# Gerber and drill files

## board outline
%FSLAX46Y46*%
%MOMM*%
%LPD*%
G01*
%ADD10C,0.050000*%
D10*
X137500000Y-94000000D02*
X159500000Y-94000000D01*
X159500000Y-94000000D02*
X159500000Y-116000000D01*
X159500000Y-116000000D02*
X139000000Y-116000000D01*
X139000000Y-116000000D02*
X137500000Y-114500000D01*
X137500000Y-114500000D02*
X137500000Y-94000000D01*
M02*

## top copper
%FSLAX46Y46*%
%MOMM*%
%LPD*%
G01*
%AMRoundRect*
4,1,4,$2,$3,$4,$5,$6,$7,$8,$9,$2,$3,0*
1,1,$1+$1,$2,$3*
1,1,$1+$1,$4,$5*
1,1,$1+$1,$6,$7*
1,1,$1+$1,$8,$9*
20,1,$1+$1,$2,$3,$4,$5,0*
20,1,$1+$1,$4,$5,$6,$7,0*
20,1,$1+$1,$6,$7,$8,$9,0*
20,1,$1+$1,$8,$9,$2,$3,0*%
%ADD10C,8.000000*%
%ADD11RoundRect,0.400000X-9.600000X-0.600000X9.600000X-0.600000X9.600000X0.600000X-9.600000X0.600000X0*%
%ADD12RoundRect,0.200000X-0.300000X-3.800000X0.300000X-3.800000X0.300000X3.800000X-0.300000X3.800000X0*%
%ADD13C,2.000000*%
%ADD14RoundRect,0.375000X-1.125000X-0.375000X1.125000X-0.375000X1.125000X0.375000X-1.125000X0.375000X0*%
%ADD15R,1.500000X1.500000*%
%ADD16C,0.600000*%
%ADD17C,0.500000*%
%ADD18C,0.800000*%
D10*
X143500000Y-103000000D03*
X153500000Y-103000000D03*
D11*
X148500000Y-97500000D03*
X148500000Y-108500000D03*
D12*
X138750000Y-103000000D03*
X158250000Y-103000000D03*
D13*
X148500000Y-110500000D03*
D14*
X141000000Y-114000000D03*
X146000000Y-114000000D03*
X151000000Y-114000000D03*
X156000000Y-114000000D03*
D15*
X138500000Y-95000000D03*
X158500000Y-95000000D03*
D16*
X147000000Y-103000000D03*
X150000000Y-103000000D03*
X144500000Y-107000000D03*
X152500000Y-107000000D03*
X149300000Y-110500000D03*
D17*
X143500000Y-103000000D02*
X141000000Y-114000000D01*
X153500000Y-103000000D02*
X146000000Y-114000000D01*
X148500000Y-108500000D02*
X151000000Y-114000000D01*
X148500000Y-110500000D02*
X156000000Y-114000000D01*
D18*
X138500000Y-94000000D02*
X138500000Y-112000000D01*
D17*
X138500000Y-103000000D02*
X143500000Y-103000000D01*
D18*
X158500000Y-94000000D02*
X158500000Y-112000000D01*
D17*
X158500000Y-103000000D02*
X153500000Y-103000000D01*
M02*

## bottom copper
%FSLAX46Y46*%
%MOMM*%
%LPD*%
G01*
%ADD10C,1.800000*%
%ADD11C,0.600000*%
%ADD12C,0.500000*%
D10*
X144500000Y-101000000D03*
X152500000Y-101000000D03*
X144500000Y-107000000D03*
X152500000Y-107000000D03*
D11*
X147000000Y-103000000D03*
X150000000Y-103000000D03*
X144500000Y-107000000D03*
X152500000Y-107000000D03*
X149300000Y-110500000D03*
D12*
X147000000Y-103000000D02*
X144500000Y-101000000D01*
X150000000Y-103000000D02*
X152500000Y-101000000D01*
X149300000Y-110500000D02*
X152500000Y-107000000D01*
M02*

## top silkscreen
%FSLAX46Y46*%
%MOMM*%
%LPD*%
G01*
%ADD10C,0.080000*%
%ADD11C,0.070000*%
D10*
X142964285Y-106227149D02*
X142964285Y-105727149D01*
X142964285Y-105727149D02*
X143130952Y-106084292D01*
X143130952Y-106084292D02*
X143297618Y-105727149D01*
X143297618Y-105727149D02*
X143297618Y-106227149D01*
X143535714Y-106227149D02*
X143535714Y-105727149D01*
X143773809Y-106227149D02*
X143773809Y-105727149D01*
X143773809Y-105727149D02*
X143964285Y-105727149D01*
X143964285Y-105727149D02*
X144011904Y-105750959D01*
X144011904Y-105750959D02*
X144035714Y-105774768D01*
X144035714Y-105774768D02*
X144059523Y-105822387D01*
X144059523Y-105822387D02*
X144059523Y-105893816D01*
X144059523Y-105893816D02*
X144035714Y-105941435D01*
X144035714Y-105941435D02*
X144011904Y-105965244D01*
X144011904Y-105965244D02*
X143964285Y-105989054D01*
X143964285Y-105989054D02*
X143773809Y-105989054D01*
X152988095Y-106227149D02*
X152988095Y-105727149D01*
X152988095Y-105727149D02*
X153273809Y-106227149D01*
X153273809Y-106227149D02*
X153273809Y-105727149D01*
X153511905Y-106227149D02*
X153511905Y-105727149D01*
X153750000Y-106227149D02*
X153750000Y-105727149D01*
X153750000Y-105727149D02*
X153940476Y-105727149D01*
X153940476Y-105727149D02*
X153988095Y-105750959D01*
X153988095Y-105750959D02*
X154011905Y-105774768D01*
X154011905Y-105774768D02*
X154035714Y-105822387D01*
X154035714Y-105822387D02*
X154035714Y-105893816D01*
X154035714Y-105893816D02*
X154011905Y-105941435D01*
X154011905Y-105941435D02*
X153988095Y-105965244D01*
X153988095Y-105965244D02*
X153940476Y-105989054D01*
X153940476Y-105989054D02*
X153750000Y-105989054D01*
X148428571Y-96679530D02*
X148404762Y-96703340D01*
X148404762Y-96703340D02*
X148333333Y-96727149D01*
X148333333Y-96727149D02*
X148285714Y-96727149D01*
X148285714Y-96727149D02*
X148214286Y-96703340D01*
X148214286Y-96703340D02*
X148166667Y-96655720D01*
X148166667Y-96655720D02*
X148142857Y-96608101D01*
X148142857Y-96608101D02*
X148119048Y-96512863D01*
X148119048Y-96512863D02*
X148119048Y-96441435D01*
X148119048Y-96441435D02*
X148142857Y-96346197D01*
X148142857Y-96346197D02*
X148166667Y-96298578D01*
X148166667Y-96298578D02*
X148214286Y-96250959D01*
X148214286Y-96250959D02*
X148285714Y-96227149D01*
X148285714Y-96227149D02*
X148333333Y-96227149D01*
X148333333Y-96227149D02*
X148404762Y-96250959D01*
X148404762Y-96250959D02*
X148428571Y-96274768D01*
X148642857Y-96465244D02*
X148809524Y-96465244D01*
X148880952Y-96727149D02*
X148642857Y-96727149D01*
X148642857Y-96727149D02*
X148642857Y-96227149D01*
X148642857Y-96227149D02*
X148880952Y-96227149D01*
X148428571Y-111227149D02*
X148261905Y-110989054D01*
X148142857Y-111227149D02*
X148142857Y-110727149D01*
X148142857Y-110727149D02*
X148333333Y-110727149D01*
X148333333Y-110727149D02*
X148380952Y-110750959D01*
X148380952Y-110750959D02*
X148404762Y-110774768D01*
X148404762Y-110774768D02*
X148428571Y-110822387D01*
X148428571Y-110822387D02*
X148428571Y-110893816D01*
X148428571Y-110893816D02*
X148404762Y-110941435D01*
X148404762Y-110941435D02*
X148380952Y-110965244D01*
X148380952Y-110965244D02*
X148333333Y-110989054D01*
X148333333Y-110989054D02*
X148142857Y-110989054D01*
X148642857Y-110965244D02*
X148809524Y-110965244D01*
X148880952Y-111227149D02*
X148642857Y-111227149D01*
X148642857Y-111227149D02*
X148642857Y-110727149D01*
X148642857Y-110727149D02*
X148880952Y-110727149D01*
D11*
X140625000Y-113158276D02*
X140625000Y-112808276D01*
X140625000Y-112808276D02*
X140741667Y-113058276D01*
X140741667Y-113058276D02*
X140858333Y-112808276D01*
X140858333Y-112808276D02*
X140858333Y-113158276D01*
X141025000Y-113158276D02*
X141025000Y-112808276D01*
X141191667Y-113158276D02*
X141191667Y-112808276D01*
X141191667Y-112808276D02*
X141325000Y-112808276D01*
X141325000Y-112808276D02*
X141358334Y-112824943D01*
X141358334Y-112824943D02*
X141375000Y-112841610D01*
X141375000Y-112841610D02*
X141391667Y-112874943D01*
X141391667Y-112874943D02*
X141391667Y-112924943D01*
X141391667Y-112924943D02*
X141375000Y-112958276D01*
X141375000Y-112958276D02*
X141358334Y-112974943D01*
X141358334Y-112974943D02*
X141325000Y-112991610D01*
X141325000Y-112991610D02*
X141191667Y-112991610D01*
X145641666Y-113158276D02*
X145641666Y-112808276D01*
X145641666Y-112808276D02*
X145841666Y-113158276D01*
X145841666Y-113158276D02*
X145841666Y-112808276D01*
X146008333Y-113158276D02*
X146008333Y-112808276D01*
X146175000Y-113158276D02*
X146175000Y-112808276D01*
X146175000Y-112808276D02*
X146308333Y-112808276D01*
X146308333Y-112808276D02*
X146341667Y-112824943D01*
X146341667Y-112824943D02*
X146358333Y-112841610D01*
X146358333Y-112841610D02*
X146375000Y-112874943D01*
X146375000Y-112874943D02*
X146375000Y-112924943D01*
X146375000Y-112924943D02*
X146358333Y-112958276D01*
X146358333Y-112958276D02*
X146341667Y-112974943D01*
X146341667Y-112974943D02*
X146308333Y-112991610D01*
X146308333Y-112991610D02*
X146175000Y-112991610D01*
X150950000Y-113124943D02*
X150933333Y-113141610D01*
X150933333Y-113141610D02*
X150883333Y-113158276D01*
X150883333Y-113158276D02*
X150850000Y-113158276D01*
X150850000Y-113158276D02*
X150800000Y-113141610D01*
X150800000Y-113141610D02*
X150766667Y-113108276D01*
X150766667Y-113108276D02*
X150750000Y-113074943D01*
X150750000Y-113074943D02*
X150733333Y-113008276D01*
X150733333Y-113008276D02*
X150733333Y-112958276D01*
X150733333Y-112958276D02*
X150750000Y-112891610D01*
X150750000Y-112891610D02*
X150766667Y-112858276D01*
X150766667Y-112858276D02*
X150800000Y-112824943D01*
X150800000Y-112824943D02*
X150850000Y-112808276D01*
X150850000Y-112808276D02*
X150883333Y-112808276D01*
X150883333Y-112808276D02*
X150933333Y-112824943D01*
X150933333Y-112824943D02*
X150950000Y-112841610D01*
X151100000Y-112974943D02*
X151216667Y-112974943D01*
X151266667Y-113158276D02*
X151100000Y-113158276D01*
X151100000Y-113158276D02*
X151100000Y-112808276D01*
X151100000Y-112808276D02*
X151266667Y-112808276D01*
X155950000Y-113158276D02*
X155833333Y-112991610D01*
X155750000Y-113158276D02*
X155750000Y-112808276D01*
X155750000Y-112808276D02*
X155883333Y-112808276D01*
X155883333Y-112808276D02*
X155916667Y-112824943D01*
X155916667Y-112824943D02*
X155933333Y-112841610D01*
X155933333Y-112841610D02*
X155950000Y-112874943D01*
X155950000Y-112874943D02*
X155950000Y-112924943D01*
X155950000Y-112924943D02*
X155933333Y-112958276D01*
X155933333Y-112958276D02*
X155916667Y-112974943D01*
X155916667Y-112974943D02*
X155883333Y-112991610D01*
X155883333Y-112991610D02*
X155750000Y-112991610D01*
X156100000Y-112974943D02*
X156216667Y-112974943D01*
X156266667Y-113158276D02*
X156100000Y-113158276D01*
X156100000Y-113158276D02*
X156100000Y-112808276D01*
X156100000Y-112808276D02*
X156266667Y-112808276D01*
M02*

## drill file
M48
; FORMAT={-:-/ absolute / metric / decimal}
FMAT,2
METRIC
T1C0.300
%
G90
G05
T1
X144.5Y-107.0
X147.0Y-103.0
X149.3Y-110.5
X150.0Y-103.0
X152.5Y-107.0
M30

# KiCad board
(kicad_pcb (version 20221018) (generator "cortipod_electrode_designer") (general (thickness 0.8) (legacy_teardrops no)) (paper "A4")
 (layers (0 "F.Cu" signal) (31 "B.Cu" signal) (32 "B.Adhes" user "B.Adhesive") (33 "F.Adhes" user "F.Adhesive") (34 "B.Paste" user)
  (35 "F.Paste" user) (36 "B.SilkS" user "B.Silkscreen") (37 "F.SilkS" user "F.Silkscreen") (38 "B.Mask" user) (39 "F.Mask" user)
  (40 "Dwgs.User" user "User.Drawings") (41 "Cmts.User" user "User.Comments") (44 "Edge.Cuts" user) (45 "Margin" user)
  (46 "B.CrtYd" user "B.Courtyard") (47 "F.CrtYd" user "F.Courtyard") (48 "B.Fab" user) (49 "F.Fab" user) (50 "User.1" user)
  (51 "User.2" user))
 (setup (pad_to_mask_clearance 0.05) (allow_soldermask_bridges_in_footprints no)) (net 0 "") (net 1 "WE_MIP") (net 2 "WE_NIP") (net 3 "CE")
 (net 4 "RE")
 (gr_line (start 137.5 94) (end 159.5 94) (layer "Edge.Cuts") (width 0.05))
 (gr_line (start 159.5 94) (end 159.5 116) (layer "Edge.Cuts") (width 0.05))
 (gr_line (start 159.5 116) (end 139 116) (layer "Edge.Cuts") (width 0.05))
 (gr_line (start 139 116) (end 137.5 114.5) (layer "Edge.Cuts") (width 0.05))
 (gr_line (start 137.5 114.5) (end 137.5 94) (layer "Edge.Cuts") (width 0.05))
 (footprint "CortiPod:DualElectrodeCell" (layer "F.Cu") (at 148.5 103)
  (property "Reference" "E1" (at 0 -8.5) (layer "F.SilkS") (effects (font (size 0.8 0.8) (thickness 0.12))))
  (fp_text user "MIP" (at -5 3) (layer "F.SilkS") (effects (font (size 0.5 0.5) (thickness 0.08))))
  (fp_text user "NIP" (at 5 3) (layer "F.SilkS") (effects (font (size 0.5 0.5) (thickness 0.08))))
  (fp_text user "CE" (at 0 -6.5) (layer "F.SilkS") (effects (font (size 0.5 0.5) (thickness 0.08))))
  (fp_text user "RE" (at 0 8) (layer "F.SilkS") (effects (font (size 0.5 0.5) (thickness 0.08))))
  (pad "1" smd circle (at -5 0) (size 8 8) (layers "F.Cu" "F.Mask") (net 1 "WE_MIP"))
  (pad "2" smd circle (at 5 0) (size 8 8) (layers "F.Cu" "F.Mask") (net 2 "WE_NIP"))
  (pad "3T" smd roundrect (at 0 -5.5) (size 20 2) (layers "F.Cu" "F.Mask") (roundrect_rratio 0.2) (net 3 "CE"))
  (pad "3B" smd roundrect (at 0 5.5) (size 20 2) (layers "F.Cu" "F.Mask") (roundrect_rratio 0.2) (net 3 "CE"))
  (pad "3L" smd roundrect (at -9.75 0) (size 1 8) (layers "F.Cu" "F.Mask") (roundrect_rratio 0.2) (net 3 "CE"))
  (pad "3R" smd roundrect (at 9.75 0) (size 1 8) (layers "F.Cu" "F.Mask") (roundrect_rratio 0.2) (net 3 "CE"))
  (pad "4" smd circle (at 0 7.5) (size 2 2) (layers "F.Cu" "F.Mask" "F.Paste") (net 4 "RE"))
  (pad "5" smd circle (at -4 -2) (size 1.8 1.8) (layers "B.Cu" "B.Mask") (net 1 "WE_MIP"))
  (pad "6" smd circle (at 4 -2) (size 1.8 1.8) (layers "B.Cu" "B.Mask") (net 2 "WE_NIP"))
  (pad "7" smd circle (at -4 4) (size 1.8 1.8) (layers "B.Cu" "B.Mask") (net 3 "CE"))
  (pad "8" smd circle (at 4 4) (size 1.8 1.8) (layers "B.Cu" "B.Mask") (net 4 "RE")))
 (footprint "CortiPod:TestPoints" (layer "F.Cu") (at 148.5 114)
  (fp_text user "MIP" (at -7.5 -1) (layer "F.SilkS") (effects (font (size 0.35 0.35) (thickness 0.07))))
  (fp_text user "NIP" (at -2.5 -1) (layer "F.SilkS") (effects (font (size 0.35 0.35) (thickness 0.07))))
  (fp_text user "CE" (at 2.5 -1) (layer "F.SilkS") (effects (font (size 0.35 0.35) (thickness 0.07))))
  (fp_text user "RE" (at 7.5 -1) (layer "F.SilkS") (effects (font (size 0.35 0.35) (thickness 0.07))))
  (pad "TP1" smd roundrect (at -7.5 0) (size 3 1.5) (layers "F.Cu" "F.Mask") (roundrect_rratio 0.25) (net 1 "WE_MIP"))
  (pad "TP2" smd roundrect (at -2.5 0) (size 3 1.5) (layers "F.Cu" "F.Mask") (roundrect_rratio 0.25) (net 2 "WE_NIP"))
  (pad "TP3" smd roundrect (at 2.5 0) (size 3 1.5) (layers "F.Cu" "F.Mask") (roundrect_rratio 0.25) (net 3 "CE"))
  (pad "TP4" smd roundrect (at 7.5 0) (size 3 1.5) (layers "F.Cu" "F.Mask") (roundrect_rratio 0.25) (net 4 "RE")))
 (via (at 147 103) (size 0.6) (drill 0.3) (layers "F.Cu" "B.Cu") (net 1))
 (via (at 150 103) (size 0.6) (drill 0.3) (layers "F.Cu" "B.Cu") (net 2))
 (via (at 144.5 107) (size 0.6) (drill 0.3) (layers "F.Cu" "B.Cu") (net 3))
 (via (at 152.5 107) (size 0.6) (drill 0.3) (layers "F.Cu" "B.Cu") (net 3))
 (via (at 149.3 110.5) (size 0.6) (drill 0.3) (layers "F.Cu" "B.Cu") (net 4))
 (segment (start 147 103) (end 144.5 101) (width 0.5) (layer "B.Cu") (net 1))
 (segment (start 150 103) (end 152.5 101) (width 0.5) (layer "B.Cu") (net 2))
 (segment (start 149.3 110.5) (end 152.5 107) (width 0.5) (layer "B.Cu") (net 4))
 (segment (start 143.5 103) (end 141 114) (width 0.5) (layer "F.Cu") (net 1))
 (segment (start 153.5 103) (end 146 114) (width 0.5) (layer "F.Cu") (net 2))
 (segment (start 148.5 108.5) (end 151 114) (width 0.5) (layer "F.Cu") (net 3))
 (segment (start 148.5 110.5) (end 156 114) (width 0.5) (layer "F.Cu") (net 4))
 (segment (start 138.5 94) (end 138.5 112) (width 0.8) (layer "F.Cu") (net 1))
 (segment (start 138.5 103) (end 143.5 103) (width 0.5) (layer "F.Cu") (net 1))
 (segment (start 158.5 94) (end 158.5 112) (width 0.8) (layer "F.Cu") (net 2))
 (segment (start 158.5 103) (end 153.5 103) (width 0.5) (layer "F.Cu") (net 2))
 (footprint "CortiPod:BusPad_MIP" (layer "F.Cu") (at 138.5 95)
  (pad "MIP_BUS" smd rect (at 0 0) (size 1.5 1.5) (layers "F.Cu" "F.Mask") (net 1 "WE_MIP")))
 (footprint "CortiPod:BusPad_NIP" (layer "F.Cu") (at 158.5 95)
  (pad "NIP_BUS" smd rect (at 0 0) (size 1.5 1.5) (layers "F.Cu" "F.Mask") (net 2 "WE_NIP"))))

